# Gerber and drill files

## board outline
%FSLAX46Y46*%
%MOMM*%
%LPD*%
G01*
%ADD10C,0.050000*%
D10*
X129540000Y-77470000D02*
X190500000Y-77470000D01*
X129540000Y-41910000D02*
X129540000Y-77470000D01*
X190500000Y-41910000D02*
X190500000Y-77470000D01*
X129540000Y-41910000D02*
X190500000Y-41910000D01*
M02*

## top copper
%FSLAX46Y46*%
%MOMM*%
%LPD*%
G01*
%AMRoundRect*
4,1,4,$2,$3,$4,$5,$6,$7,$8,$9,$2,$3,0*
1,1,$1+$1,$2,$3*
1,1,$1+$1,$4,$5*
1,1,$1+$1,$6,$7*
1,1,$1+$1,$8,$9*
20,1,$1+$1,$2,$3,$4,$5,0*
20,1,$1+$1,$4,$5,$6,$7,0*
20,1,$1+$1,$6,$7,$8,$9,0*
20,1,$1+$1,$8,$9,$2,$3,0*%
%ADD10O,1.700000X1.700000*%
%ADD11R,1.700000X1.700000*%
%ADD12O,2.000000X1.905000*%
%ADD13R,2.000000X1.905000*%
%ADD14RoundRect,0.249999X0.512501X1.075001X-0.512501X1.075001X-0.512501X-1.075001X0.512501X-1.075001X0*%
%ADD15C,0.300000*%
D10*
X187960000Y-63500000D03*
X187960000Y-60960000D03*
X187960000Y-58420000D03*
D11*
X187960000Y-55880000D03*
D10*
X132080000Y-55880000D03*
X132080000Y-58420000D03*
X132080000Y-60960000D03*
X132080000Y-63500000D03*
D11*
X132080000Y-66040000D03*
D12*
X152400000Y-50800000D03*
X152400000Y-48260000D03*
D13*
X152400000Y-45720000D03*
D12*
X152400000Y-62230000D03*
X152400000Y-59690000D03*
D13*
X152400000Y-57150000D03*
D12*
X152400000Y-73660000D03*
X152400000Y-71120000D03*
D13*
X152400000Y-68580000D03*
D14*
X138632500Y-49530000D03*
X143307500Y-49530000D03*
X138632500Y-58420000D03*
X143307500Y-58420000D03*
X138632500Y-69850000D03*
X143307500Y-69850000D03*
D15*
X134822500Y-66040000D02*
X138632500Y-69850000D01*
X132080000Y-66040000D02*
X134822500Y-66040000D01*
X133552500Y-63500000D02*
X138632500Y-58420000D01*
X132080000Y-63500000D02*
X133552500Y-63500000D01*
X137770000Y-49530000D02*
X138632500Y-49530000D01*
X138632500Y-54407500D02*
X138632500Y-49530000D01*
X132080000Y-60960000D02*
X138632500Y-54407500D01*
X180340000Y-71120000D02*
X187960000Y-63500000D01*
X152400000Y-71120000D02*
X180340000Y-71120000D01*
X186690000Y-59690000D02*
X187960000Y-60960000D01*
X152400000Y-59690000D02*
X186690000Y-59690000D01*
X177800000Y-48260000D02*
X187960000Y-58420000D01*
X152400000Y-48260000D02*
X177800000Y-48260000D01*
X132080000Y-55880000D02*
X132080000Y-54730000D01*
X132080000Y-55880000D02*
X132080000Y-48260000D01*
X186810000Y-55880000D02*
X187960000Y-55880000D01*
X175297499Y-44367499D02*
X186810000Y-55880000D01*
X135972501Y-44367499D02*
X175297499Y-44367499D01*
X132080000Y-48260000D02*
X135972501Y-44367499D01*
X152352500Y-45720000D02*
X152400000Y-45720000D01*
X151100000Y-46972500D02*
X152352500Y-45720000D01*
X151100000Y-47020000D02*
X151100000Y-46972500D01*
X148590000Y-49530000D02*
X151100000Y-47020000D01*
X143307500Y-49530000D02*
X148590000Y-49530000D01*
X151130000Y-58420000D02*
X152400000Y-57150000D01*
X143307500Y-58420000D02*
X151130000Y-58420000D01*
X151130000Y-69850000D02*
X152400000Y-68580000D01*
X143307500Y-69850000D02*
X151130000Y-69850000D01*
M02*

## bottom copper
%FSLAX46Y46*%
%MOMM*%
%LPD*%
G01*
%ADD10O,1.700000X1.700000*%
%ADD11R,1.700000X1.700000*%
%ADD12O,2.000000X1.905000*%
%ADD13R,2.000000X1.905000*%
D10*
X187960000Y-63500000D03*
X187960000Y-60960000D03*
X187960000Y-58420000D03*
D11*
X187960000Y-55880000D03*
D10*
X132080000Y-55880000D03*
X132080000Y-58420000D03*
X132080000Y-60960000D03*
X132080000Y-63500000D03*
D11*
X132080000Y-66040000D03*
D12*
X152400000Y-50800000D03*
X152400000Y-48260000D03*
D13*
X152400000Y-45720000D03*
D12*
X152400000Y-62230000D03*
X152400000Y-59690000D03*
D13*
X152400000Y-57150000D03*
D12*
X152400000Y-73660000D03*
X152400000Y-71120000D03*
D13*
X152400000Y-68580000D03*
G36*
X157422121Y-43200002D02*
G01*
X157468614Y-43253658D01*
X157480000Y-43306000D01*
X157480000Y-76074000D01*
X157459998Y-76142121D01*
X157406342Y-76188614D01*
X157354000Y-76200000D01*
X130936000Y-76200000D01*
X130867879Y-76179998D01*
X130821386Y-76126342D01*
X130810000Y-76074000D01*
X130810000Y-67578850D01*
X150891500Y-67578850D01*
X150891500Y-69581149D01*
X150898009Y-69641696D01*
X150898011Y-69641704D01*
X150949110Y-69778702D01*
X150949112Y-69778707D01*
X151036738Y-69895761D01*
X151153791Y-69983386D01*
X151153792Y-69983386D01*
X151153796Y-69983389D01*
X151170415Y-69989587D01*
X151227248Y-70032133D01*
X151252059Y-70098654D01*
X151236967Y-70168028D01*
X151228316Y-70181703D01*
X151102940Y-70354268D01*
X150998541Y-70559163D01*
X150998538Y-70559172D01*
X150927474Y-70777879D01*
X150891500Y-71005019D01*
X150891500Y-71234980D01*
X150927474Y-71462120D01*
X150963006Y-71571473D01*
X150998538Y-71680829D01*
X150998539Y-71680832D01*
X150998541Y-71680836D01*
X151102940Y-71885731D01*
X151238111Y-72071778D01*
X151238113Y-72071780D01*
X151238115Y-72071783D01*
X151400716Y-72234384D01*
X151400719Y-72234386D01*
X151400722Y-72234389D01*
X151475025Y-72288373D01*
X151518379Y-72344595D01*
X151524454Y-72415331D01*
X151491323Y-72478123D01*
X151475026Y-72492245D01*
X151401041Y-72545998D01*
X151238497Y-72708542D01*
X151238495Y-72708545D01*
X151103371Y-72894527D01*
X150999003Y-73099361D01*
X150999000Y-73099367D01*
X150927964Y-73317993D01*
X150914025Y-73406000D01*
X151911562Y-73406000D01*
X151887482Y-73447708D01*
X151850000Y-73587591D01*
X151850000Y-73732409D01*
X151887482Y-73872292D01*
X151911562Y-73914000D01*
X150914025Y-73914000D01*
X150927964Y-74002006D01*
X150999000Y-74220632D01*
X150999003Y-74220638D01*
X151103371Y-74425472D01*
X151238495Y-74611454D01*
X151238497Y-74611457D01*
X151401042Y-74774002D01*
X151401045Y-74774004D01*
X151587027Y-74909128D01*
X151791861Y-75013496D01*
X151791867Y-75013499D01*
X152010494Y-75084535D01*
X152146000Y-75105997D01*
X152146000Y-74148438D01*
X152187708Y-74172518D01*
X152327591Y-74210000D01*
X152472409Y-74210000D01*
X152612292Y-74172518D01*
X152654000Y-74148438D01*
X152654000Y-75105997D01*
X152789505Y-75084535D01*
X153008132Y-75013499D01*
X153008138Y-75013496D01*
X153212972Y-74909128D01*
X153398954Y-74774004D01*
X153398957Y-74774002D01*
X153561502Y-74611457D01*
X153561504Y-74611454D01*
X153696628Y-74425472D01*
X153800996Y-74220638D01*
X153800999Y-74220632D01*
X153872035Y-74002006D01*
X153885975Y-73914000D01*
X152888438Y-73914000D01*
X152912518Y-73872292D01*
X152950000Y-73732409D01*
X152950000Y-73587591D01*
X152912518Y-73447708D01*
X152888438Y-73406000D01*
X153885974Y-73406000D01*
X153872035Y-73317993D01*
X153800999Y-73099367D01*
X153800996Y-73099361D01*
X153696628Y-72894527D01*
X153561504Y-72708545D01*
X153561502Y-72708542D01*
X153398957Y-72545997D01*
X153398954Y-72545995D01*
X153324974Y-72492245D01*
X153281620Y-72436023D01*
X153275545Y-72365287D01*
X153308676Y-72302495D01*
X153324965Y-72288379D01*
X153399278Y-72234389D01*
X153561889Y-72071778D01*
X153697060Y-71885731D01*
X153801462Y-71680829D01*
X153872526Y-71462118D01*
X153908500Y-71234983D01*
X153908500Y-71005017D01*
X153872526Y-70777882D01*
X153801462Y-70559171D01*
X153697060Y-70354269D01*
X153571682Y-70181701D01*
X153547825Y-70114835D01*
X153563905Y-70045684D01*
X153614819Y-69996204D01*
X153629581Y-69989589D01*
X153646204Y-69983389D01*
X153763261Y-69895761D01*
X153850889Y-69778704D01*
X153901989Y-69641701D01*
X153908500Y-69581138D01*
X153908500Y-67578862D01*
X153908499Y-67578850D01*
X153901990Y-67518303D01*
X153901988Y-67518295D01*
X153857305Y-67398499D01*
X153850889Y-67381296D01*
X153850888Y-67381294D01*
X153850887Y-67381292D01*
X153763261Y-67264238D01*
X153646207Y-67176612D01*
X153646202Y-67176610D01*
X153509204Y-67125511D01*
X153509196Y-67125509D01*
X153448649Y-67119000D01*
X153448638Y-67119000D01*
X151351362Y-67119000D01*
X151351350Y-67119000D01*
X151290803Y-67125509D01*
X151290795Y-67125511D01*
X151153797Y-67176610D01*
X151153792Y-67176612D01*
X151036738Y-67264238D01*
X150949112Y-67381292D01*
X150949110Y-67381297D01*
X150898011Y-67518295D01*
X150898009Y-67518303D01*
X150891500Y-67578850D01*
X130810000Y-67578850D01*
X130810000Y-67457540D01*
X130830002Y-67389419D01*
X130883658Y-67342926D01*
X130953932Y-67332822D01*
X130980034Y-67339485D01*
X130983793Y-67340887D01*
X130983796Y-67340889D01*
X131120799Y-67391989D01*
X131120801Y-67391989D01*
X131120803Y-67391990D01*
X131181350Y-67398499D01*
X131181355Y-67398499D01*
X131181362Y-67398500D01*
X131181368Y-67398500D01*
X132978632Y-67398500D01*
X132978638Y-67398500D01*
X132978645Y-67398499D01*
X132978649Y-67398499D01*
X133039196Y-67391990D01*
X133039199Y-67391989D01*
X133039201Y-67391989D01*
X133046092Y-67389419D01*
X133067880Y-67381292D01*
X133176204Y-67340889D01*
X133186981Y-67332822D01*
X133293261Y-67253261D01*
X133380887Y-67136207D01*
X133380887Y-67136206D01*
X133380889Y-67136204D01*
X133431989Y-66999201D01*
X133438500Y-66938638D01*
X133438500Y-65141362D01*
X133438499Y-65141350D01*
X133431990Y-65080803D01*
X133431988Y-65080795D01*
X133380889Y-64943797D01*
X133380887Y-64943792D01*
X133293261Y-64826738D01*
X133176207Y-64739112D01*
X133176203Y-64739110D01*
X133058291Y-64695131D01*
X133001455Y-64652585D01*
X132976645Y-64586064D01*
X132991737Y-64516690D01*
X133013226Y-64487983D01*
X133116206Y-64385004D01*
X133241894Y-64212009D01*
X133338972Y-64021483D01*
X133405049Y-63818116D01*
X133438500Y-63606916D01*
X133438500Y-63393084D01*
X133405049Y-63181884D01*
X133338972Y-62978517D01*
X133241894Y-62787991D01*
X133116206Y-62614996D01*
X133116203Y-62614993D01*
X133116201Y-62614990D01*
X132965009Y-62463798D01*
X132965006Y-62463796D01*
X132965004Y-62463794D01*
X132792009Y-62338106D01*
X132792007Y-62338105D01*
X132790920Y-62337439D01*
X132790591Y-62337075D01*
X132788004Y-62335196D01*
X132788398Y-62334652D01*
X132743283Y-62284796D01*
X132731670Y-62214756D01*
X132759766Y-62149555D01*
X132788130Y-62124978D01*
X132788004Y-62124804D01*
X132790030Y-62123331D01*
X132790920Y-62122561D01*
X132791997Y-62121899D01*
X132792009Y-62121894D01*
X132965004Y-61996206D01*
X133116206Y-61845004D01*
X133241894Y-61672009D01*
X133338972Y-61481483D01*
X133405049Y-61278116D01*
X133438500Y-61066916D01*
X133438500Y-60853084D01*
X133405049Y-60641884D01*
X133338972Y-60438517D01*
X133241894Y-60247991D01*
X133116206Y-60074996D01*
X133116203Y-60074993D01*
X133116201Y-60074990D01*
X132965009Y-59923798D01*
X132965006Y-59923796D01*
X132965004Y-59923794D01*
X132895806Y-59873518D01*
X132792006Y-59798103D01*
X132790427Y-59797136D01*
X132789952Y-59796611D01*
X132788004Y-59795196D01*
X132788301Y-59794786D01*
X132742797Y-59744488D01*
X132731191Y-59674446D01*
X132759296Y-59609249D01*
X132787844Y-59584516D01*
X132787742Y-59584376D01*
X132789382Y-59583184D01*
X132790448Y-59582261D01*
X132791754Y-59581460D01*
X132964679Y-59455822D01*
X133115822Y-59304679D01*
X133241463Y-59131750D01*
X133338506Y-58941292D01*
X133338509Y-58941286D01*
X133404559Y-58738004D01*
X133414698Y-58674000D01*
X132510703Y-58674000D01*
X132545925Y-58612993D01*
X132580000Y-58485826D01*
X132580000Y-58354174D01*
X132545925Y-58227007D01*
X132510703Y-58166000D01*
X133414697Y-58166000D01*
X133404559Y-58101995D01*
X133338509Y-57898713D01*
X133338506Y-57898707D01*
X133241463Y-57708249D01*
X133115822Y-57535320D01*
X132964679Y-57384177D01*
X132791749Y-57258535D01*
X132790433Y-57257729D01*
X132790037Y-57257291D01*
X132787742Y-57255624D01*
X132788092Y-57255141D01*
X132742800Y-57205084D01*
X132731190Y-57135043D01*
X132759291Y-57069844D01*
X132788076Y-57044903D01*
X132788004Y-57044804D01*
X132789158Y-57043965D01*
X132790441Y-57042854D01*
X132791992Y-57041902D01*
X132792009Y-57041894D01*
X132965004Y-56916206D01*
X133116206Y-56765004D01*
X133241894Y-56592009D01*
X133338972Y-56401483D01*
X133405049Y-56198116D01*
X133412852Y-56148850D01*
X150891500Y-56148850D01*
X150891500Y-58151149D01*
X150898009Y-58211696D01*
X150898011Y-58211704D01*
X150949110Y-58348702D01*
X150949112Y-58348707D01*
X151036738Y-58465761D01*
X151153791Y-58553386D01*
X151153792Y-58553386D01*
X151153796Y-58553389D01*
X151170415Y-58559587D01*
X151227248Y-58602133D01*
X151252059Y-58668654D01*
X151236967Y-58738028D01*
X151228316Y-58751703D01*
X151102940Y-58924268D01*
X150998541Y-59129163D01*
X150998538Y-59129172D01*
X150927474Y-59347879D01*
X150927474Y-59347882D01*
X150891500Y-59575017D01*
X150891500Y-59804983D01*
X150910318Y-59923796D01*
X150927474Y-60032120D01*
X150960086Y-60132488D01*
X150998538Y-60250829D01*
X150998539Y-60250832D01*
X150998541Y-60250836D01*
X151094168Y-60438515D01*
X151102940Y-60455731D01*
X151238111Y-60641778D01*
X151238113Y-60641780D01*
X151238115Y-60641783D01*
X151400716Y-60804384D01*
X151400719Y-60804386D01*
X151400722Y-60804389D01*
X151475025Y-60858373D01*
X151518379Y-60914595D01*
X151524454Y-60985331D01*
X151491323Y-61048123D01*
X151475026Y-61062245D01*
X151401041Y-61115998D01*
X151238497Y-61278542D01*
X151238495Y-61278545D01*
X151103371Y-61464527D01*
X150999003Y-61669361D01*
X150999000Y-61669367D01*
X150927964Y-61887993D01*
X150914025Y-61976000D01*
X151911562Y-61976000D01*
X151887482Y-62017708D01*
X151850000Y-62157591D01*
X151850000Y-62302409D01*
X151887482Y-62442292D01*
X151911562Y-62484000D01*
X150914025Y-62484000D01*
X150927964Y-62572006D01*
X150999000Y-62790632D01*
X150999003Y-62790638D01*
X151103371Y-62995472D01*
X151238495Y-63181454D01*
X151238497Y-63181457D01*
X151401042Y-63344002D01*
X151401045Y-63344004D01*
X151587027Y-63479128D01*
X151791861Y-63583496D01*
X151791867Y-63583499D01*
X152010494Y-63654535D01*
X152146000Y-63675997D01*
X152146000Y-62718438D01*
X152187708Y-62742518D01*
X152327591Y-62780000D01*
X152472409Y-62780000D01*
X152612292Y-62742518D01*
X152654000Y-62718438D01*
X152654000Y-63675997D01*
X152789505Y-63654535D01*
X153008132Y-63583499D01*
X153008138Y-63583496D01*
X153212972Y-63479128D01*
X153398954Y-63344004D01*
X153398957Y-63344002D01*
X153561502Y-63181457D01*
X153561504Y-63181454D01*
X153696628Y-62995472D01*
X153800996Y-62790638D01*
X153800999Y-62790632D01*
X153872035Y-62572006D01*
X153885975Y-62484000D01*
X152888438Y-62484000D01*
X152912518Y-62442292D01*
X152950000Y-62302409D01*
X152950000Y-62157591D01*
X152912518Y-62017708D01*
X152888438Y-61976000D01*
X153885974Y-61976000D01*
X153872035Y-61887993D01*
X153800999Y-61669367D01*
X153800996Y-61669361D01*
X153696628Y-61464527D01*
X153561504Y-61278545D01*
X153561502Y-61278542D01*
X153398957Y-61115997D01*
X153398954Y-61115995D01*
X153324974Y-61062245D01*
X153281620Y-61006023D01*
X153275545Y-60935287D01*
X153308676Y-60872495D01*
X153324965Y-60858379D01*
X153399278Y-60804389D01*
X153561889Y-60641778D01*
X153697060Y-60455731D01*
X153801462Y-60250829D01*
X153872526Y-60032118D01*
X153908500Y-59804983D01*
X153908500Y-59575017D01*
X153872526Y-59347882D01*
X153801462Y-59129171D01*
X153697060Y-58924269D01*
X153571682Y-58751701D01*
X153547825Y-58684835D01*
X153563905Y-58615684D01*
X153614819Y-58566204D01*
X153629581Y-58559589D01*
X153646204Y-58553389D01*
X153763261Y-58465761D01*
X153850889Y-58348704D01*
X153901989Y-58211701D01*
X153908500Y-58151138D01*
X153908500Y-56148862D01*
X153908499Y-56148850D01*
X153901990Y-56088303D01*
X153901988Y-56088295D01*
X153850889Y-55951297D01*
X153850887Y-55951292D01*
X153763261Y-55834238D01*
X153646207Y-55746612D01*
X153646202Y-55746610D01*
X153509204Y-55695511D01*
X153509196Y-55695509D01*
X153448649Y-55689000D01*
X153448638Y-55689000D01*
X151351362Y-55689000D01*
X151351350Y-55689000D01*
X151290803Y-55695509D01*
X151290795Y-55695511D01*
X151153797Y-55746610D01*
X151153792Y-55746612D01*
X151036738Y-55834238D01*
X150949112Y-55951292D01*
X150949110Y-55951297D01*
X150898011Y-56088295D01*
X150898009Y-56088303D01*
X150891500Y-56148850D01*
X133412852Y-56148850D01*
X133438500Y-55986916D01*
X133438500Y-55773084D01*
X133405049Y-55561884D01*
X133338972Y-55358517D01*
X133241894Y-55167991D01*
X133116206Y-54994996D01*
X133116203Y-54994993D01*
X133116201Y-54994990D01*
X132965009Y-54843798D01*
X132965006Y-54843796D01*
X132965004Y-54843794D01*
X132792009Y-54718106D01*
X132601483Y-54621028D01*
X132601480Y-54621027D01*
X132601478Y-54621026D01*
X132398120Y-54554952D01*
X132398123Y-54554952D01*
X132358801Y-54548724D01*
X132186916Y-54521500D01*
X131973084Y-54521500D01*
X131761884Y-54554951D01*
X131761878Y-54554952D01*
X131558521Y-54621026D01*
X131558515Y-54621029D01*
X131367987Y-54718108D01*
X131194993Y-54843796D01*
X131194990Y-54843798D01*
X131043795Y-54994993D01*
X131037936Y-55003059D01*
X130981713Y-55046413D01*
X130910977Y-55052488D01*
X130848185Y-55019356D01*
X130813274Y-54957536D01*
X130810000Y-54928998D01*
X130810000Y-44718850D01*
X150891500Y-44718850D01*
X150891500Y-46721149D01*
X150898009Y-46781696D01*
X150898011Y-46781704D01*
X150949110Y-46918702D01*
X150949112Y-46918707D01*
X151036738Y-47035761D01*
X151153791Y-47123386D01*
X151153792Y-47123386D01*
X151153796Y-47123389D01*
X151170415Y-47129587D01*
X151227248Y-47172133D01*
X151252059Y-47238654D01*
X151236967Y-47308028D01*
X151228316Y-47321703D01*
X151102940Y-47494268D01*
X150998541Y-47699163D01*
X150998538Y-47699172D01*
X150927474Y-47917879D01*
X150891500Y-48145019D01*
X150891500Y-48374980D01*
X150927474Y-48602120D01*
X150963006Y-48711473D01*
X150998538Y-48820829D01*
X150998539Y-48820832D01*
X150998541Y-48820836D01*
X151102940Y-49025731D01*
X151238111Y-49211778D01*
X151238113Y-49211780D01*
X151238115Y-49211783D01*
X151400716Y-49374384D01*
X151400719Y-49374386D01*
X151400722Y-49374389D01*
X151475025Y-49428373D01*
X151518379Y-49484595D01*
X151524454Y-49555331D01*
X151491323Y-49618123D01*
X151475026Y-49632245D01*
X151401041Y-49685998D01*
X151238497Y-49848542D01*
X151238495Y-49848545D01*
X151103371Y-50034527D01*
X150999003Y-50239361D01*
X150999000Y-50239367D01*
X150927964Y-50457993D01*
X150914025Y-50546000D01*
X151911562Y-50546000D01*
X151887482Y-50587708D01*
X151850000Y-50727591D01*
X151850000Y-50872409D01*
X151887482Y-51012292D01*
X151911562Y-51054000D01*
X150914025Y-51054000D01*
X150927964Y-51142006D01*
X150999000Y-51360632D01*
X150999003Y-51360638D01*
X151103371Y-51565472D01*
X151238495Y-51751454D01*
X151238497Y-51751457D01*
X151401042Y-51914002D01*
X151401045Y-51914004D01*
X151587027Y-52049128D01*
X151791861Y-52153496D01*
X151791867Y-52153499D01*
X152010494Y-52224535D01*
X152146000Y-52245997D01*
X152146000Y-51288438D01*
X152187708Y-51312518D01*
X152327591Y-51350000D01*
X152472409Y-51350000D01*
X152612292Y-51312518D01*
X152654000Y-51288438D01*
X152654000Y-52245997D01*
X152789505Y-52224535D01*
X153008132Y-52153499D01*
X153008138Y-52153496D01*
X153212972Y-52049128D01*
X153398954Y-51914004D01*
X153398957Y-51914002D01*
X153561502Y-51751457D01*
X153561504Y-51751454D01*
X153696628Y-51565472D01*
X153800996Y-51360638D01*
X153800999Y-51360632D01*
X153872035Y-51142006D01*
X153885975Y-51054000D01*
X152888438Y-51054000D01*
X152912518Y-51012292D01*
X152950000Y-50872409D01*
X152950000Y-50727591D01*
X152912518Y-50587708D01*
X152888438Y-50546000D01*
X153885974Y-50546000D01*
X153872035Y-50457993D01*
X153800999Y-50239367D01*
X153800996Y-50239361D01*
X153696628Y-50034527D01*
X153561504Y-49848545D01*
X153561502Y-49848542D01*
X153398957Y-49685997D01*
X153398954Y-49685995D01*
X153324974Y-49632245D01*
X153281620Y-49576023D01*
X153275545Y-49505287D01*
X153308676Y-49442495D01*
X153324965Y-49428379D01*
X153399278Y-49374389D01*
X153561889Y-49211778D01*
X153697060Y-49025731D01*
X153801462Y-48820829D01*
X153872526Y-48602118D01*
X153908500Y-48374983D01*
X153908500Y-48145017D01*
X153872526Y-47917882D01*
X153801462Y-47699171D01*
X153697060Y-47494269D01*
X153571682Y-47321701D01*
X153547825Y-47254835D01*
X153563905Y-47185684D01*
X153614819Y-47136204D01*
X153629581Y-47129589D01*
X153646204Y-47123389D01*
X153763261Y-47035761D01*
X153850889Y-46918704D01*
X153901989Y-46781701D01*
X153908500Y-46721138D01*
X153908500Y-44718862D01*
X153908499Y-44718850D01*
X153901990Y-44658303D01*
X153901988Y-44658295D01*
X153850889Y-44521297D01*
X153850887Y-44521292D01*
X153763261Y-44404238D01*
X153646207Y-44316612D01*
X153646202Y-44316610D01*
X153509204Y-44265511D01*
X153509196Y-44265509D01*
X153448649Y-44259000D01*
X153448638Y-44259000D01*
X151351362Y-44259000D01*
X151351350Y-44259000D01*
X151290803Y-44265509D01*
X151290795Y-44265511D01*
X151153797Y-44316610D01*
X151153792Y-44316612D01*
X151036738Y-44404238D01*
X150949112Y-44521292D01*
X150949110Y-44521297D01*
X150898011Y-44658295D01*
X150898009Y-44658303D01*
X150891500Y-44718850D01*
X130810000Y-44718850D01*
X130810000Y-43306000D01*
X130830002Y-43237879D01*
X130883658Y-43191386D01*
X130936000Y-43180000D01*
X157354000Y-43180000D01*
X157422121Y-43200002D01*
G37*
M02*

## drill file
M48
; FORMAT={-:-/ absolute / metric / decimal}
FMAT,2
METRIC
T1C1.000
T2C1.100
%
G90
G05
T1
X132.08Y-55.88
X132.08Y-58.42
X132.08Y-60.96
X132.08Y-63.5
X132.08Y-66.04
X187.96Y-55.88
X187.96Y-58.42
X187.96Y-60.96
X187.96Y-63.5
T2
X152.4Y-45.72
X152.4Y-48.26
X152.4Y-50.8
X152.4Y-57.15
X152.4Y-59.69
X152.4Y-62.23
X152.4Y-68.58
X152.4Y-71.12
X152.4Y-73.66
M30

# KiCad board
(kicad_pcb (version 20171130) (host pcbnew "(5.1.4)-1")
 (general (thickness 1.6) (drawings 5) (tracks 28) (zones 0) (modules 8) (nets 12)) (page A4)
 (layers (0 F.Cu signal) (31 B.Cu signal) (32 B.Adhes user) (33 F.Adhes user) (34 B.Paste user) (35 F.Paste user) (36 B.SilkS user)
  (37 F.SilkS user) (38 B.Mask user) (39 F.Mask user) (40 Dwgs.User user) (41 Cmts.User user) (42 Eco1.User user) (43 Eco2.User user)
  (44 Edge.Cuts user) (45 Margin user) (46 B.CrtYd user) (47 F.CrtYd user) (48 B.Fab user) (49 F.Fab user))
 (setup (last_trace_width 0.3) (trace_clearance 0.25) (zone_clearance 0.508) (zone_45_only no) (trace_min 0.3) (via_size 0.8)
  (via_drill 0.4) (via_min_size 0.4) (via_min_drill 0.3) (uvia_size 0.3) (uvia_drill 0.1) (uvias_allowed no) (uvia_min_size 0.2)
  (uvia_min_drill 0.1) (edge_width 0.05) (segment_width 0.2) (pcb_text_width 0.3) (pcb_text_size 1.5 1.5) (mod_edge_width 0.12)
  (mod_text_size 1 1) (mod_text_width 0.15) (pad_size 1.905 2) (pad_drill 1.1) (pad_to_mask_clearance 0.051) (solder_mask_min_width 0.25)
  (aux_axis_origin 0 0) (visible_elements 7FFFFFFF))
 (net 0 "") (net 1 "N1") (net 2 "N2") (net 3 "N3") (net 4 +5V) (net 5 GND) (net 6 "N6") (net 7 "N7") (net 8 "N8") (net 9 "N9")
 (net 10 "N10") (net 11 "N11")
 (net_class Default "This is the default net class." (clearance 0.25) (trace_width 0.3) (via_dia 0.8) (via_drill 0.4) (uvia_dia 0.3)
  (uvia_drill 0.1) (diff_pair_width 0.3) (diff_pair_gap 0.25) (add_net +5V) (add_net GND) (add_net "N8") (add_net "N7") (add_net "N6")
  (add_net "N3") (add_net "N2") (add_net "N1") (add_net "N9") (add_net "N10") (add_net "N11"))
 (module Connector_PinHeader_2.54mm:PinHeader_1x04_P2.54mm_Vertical (layer F.Cu) (at 187.96 55.88)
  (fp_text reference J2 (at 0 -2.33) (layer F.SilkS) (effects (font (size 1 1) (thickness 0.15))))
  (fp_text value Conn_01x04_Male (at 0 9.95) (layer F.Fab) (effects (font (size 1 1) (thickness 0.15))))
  (pad 4 thru_hole oval (at 0 7.62) (size 1.7 1.7) (drill 1) (layers *.Cu *.Mask) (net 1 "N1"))
  (pad 3 thru_hole oval (at 0 5.08) (size 1.7 1.7) (drill 1) (layers *.Cu *.Mask) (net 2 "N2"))
  (pad 2 thru_hole oval (at 0 2.54) (size 1.7 1.7) (drill 1) (layers *.Cu *.Mask) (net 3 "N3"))
  (pad 1 thru_hole rect (at 0 0) (size 1.7 1.7) (drill 1) (layers *.Cu *.Mask) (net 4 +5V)))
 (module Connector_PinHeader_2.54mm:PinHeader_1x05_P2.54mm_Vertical (layer F.Cu) (at 132.08 66.04 180)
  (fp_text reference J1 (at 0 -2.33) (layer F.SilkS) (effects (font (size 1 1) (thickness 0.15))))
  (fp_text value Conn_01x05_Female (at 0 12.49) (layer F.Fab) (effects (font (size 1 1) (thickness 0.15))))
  (pad 5 thru_hole oval (at 0 10.16 180) (size 1.7 1.7) (drill 1) (layers *.Cu *.Mask) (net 4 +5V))
  (pad 4 thru_hole oval (at 0 7.62 180) (size 1.7 1.7) (drill 1) (layers *.Cu *.Mask) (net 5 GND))
  (pad 3 thru_hole oval (at 0 5.08 180) (size 1.7 1.7) (drill 1) (layers *.Cu *.Mask) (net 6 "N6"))
  (pad 2 thru_hole oval (at 0 2.54 180) (size 1.7 1.7) (drill 1) (layers *.Cu *.Mask) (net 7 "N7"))
  (pad 1 thru_hole rect (at 0 0 180) (size 1.7 1.7) (drill 1) (layers *.Cu *.Mask) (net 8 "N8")))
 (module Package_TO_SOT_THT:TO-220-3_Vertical (layer F.Cu) (at 152.4 45.72 270)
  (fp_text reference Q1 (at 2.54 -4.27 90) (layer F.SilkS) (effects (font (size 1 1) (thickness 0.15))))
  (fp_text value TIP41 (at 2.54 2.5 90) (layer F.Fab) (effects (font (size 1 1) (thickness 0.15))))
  (pad 3 thru_hole oval (at 5.08 0 270) (size 1.905 2) (drill 1.1) (layers *.Cu *.Mask) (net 5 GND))
  (pad 2 thru_hole oval (at 2.54 0 270) (size 1.905 2) (drill 1.1) (layers *.Cu *.Mask) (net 3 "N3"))
  (pad 1 thru_hole rect (at 0 0 270) (size 1.905 2) (drill 1.1) (layers *.Cu *.Mask) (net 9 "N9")))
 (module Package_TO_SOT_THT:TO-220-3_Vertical (layer F.Cu) (at 152.4 57.15 270)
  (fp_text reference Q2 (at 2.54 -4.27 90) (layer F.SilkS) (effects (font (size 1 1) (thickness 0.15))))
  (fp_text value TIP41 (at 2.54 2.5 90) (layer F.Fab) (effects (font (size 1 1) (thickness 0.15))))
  (pad 3 thru_hole oval (at 5.08 0 270) (size 1.905 2) (drill 1.1) (layers *.Cu *.Mask) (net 5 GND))
  (pad 2 thru_hole oval (at 2.54 0 270) (size 1.905 2) (drill 1.1) (layers *.Cu *.Mask) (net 2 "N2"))
  (pad 1 thru_hole rect (at 0 0 270) (size 1.905 2) (drill 1.1) (layers *.Cu *.Mask) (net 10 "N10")))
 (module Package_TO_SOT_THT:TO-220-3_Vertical (layer F.Cu) (at 152.4 68.58 270)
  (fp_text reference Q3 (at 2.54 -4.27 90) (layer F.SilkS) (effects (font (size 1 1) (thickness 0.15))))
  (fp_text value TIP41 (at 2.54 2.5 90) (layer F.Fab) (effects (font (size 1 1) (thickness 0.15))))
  (pad 3 thru_hole oval (at 5.08 0 270) (size 1.905 2) (drill 1.1) (layers *.Cu *.Mask) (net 5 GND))
  (pad 2 thru_hole oval (at 2.54 0 270) (size 1.905 2) (drill 1.1) (layers *.Cu *.Mask) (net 1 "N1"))
  (pad 1 thru_hole rect (at 0 0 270) (size 1.905 2) (drill 1.1) (layers *.Cu *.Mask) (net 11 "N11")))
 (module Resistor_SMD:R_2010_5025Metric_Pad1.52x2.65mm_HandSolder (layer F.Cu) (at 140.97 49.53 180)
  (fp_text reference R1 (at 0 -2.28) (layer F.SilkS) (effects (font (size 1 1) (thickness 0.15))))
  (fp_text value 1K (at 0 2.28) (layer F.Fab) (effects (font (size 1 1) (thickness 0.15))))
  (pad 2 smd roundrect (at 2.3375 0 180) (size 1.525 2.65) (layers F.Cu F.Paste F.Mask) (roundrect_rratio 0.163934) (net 6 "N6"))
  (pad 1 smd roundrect (at -2.3375 0 180) (size 1.525 2.65) (layers F.Cu F.Paste F.Mask) (roundrect_rratio 0.163934) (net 9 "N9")))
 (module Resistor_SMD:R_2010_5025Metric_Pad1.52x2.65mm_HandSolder (layer F.Cu) (at 140.97 58.42 180)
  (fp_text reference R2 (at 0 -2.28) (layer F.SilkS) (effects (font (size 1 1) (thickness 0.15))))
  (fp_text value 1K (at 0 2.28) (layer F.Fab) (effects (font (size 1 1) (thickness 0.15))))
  (pad 2 smd roundrect (at 2.3375 0 180) (size 1.525 2.65) (layers F.Cu F.Paste F.Mask) (roundrect_rratio 0.163934) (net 7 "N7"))
  (pad 1 smd roundrect (at -2.3375 0 180) (size 1.525 2.65) (layers F.Cu F.Paste F.Mask) (roundrect_rratio 0.163934) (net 10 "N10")))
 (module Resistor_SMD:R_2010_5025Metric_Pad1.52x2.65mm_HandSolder (layer F.Cu) (at 140.97 69.85 180)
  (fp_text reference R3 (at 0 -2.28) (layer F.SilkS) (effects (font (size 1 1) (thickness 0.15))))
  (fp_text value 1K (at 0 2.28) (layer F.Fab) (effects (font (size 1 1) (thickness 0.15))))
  (pad 2 smd roundrect (at 2.3375 0 180) (size 1.525 2.65) (layers F.Cu F.Paste F.Mask) (roundrect_rratio 0.163934) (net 8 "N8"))
  (pad 1 smd roundrect (at -2.3375 0 180) (size 1.525 2.65) (layers F.Cu F.Paste F.Mask) (roundrect_rratio 0.163934) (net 11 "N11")))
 (gr_line (start 129.54 77.47) (end 190.5 77.47) (layer Edge.Cuts) (width 0.05))
 (gr_line (start 129.54 41.91) (end 129.54 77.47) (layer Edge.Cuts) (width 0.05))
 (gr_line (start 190.5 41.91) (end 190.5 77.47) (layer Edge.Cuts) (width 0.05))
 (gr_line (start 129.54 41.91) (end 190.5 41.91) (layer Edge.Cuts) (width 0.05))
 (segment (start 134.8225 66.04) (end 138.6325 69.85) (width 0.3) (layer F.Cu) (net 8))
 (segment (start 132.08 66.04) (end 134.8225 66.04) (width 0.3) (layer F.Cu) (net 8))
 (segment (start 133.5525 63.5) (end 138.6325 58.42) (width 0.3) (layer F.Cu) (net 7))
 (segment (start 132.08 63.5) (end 133.5525 63.5) (width 0.3) (layer F.Cu) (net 7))
 (segment (start 137.77 49.53) (end 138.6325 49.53) (width 0.3) (layer F.Cu) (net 6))
 (segment (start 138.6325 54.4075) (end 138.6325 49.53) (width 0.3) (layer F.Cu) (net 6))
 (segment (start 132.08 60.96) (end 138.6325 54.4075) (width 0.3) (layer F.Cu) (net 6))
 (segment (start 180.34 71.12) (end 187.96 63.5) (width 0.3) (layer F.Cu) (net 1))
 (segment (start 152.4 71.12) (end 180.34 71.12) (width 0.3) (layer F.Cu) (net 1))
 (segment (start 186.69 59.69) (end 187.96 60.96) (width 0.3) (layer F.Cu) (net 2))
 (segment (start 152.4 59.69) (end 186.69 59.69) (width 0.3) (layer F.Cu) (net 2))
 (segment (start 177.8 48.26) (end 187.96 58.42) (width 0.3) (layer F.Cu) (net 3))
 (segment (start 152.4 48.26) (end 177.8 48.26) (width 0.3) (layer F.Cu) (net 3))
 (segment (start 132.08 55.88) (end 132.08 54.73) (width 0.3) (layer F.Cu) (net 4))
 (segment (start 132.08 55.88) (end 132.08 48.26) (width 0.3) (layer F.Cu) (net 4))
 (segment (start 186.81 55.88) (end 187.96 55.88) (width 0.3) (layer F.Cu) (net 4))
 (segment (start 175.297499 44.367499) (end 186.81 55.88) (width 0.3) (layer F.Cu) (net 4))
 (segment (start 135.972501 44.367499) (end 175.297499 44.367499) (width 0.3) (layer F.Cu) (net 4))
 (segment (start 132.08 48.26) (end 135.972501 44.367499) (width 0.3) (layer F.Cu) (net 4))
 (segment (start 152.3525 45.72) (end 152.4 45.72) (width 0.3) (layer F.Cu) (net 9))
 (segment (start 151.1 46.9725) (end 152.3525 45.72) (width 0.3) (layer F.Cu) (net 9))
 (segment (start 151.1 47.02) (end 151.1 46.9725) (width 0.3) (layer F.Cu) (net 9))
 (segment (start 148.59 49.53) (end 151.1 47.02) (width 0.3) (layer F.Cu) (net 9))
 (segment (start 143.3075 49.53) (end 148.59 49.53) (width 0.3) (layer F.Cu) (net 9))
 (segment (start 151.13 58.42) (end 152.4 57.15) (width 0.3) (layer F.Cu) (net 10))
 (segment (start 143.3075 58.42) (end 151.13 58.42) (width 0.3) (layer F.Cu) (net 10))
 (segment (start 151.13 69.85) (end 152.4 68.58) (width 0.3) (layer F.Cu) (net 11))
 (segment (start 143.3075 69.85) (end 151.13 69.85) (width 0.3) (layer F.Cu) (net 11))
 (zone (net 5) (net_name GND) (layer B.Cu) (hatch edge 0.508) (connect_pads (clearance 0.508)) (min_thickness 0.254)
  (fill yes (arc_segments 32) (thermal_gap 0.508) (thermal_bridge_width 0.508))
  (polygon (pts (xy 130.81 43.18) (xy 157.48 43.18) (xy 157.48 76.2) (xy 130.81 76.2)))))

